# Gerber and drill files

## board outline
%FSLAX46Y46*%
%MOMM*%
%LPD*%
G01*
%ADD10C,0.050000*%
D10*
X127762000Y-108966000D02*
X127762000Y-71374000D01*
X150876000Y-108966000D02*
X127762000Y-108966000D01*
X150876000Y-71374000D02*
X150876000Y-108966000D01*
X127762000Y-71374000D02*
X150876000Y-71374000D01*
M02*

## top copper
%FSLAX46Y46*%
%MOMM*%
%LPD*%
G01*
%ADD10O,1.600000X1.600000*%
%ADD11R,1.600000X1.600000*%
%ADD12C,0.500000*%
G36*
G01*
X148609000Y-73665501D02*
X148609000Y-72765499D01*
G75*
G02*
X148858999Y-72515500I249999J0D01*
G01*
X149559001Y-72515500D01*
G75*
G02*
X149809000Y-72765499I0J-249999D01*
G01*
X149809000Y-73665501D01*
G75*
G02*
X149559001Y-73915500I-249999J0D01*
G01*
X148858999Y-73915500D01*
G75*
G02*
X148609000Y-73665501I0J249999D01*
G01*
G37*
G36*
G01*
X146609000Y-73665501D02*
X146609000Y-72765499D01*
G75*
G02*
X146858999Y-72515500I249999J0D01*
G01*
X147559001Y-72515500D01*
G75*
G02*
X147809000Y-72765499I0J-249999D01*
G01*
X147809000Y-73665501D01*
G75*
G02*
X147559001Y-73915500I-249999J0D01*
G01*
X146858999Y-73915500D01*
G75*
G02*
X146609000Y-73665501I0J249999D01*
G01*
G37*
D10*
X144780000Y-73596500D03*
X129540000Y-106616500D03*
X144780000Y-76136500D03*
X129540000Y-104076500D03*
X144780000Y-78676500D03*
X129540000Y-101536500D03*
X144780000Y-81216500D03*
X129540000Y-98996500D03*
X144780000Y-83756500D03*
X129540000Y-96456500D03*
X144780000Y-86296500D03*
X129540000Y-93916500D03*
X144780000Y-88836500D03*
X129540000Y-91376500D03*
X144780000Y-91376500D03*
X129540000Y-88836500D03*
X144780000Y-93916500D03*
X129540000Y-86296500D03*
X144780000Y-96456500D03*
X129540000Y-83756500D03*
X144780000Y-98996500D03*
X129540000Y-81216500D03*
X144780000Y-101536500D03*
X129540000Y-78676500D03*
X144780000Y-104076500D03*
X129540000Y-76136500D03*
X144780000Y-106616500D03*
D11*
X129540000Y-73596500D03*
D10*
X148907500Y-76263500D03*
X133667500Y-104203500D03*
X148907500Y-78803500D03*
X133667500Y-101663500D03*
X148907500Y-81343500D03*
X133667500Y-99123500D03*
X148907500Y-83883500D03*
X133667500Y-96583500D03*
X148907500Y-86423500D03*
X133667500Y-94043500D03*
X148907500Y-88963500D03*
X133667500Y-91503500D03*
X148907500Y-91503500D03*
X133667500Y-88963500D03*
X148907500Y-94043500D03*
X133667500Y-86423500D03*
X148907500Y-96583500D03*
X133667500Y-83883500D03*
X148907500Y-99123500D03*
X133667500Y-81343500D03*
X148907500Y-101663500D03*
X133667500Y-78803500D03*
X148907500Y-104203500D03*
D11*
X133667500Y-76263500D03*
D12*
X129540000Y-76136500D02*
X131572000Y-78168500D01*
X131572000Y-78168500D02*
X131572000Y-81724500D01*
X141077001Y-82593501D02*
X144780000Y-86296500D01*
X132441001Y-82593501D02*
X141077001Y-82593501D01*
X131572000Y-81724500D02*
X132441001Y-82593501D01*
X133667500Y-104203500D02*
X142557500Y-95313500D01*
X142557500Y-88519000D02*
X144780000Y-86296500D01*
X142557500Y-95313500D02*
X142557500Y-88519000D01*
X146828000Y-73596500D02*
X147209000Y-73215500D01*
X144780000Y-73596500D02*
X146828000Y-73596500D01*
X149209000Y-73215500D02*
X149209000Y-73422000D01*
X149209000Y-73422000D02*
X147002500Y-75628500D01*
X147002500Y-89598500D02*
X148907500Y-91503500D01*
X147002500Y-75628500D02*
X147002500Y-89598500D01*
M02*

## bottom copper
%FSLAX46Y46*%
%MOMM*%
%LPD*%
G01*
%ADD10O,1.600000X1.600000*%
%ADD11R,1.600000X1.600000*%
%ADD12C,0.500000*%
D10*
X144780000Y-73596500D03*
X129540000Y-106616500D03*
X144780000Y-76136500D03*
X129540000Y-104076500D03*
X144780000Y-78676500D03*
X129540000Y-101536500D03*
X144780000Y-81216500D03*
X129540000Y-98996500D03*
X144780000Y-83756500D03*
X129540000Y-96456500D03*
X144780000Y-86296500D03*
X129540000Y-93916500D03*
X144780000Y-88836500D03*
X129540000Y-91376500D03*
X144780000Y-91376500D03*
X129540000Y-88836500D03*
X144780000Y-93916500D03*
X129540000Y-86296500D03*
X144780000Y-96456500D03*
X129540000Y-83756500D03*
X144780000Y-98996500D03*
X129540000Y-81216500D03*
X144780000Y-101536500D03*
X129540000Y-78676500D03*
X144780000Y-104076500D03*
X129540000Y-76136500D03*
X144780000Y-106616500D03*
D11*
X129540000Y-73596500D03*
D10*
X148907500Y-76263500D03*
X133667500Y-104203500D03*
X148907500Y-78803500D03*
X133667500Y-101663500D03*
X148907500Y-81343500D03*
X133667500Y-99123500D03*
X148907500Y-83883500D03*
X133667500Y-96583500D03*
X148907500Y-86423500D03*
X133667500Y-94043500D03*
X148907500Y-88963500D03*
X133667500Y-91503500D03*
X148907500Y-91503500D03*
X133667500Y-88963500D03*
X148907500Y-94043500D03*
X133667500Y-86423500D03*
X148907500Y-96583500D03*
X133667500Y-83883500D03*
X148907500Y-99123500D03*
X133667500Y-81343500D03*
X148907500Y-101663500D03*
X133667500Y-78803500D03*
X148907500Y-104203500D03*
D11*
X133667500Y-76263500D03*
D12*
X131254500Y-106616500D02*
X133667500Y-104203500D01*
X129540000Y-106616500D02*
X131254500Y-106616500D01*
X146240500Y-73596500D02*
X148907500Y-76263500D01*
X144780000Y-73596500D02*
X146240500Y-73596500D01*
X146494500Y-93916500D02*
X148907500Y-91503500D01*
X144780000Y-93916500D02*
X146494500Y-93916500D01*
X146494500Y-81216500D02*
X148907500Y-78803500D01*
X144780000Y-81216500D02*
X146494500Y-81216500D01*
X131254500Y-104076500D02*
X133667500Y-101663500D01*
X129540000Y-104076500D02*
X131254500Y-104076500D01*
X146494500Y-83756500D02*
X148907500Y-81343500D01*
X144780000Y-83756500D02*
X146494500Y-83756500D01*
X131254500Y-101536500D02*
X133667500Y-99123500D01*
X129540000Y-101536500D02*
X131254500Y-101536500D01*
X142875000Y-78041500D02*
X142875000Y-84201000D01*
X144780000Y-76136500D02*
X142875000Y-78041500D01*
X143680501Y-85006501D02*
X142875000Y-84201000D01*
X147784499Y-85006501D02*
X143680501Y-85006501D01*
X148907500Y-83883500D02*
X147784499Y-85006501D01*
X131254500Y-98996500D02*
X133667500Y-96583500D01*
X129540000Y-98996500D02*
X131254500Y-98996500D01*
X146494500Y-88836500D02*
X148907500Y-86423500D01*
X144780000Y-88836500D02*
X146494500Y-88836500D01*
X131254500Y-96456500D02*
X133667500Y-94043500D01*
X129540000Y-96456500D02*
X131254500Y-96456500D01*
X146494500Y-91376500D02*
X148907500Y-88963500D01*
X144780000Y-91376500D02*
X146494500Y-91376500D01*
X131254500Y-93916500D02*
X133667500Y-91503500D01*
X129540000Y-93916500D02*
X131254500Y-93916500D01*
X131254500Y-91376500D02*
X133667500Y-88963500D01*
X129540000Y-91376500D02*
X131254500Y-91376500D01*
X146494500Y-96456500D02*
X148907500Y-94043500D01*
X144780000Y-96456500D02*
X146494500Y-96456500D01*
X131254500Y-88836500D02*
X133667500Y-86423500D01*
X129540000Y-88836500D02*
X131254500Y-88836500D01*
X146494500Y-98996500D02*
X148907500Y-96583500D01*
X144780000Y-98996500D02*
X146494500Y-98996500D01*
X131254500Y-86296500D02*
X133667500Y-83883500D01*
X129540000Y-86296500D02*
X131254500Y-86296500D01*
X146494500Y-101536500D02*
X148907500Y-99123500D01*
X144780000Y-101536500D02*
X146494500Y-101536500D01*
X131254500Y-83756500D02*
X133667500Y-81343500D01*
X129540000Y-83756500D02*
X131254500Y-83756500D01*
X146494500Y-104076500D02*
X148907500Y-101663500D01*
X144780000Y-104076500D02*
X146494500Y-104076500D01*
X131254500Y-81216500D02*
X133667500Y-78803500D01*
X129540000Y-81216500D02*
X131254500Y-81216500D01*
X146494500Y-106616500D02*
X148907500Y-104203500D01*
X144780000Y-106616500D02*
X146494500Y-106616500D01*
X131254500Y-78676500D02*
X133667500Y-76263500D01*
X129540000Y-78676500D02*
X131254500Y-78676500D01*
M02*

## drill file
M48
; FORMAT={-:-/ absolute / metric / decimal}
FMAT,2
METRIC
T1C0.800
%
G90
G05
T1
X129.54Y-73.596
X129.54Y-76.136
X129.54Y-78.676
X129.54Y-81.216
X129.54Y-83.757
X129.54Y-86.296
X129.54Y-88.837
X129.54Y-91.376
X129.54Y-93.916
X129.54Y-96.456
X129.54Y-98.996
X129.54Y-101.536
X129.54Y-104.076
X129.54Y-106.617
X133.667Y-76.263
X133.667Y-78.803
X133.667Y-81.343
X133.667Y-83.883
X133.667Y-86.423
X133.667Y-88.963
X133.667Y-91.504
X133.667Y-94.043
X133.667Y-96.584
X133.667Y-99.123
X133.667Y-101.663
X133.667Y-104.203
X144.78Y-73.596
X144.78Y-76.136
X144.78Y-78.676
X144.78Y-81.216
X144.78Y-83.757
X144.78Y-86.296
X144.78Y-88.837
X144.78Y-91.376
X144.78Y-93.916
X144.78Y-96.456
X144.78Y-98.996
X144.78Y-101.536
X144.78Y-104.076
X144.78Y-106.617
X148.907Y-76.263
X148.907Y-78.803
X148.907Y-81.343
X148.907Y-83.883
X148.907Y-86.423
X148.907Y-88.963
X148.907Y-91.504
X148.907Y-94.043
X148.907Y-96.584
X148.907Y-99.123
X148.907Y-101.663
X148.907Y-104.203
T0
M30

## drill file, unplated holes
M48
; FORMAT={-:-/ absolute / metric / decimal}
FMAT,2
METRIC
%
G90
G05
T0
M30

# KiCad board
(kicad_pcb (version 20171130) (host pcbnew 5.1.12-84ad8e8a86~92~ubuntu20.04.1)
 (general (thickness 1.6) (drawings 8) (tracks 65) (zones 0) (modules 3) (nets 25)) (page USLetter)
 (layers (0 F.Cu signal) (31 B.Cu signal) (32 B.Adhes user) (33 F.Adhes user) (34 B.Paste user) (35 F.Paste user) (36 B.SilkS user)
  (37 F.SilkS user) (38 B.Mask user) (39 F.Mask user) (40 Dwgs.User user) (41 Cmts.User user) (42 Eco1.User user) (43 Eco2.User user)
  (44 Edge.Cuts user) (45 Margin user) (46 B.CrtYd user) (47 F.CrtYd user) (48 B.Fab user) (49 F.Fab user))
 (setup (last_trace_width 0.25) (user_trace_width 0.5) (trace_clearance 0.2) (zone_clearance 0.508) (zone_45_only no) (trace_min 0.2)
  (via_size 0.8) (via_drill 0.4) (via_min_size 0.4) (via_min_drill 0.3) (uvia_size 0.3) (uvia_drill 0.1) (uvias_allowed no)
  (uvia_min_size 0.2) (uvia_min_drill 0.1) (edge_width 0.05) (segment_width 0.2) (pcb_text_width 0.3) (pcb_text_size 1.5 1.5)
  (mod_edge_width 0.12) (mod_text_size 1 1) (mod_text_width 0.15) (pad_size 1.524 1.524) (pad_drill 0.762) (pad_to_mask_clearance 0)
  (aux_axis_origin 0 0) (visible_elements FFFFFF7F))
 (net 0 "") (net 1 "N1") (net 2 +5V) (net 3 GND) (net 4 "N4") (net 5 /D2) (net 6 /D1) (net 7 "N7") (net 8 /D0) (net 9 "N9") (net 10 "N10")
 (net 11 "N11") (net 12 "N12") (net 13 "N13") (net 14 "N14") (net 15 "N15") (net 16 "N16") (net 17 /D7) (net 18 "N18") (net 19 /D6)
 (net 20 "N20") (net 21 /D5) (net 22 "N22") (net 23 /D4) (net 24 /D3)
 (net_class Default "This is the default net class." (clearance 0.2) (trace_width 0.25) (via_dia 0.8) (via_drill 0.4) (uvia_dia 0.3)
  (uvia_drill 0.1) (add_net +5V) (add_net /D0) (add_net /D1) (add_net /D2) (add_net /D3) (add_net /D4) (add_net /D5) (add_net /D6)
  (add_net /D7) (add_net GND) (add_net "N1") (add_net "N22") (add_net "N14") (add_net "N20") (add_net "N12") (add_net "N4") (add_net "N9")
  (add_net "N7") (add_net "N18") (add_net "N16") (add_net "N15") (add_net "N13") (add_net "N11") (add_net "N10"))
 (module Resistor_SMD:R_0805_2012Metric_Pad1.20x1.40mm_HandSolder (layer F.Cu) (at 148.209 73.2155)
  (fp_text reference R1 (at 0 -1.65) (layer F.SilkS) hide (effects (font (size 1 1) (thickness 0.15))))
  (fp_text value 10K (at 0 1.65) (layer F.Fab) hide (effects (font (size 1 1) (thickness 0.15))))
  (pad 2 smd roundrect (at 1 0) (size 1.2 1.4) (layers F.Cu F.Paste F.Mask) (roundrect_rratio 0.2083325) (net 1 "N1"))
  (pad 1 smd roundrect (at -1 0) (size 1.2 1.4) (layers F.Cu F.Paste F.Mask) (roundrect_rratio 0.2083325) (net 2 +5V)))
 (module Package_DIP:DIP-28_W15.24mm (layer F.Cu) (at 129.54 73.5965)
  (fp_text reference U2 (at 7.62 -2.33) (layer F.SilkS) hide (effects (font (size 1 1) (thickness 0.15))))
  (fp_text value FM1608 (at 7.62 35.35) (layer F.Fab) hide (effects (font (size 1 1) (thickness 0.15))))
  (pad 28 thru_hole oval (at 15.24 0) (size 1.6 1.6) (drill 0.8) (layers *.Cu *.Mask) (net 2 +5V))
  (pad 14 thru_hole oval (at 0 33.02) (size 1.6 1.6) (drill 0.8) (layers *.Cu *.Mask) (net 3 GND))
  (pad 27 thru_hole oval (at 15.24 2.54) (size 1.6 1.6) (drill 0.8) (layers *.Cu *.Mask) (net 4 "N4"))
  (pad 13 thru_hole oval (at 0 30.48) (size 1.6 1.6) (drill 0.8) (layers *.Cu *.Mask) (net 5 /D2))
  (pad 26 thru_hole oval (at 15.24 5.08) (size 1.6 1.6) (drill 0.8) (layers *.Cu *.Mask))
  (pad 12 thru_hole oval (at 0 27.94) (size 1.6 1.6) (drill 0.8) (layers *.Cu *.Mask) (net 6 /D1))
  (pad 25 thru_hole oval (at 15.24 7.62) (size 1.6 1.6) (drill 0.8) (layers *.Cu *.Mask) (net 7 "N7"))
  (pad 11 thru_hole oval (at 0 25.4) (size 1.6 1.6) (drill 0.8) (layers *.Cu *.Mask) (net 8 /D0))
  (pad 24 thru_hole oval (at 15.24 10.16) (size 1.6 1.6) (drill 0.8) (layers *.Cu *.Mask) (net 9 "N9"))
  (pad 10 thru_hole oval (at 0 22.86) (size 1.6 1.6) (drill 0.8) (layers *.Cu *.Mask) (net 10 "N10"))
  (pad 23 thru_hole oval (at 15.24 12.7) (size 1.6 1.6) (drill 0.8) (layers *.Cu *.Mask) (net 3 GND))
  (pad 9 thru_hole oval (at 0 20.32) (size 1.6 1.6) (drill 0.8) (layers *.Cu *.Mask) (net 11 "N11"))
  (pad 22 thru_hole oval (at 15.24 15.24) (size 1.6 1.6) (drill 0.8) (layers *.Cu *.Mask) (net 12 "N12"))
  (pad 8 thru_hole oval (at 0 17.78) (size 1.6 1.6) (drill 0.8) (layers *.Cu *.Mask) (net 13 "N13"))
  (pad 21 thru_hole oval (at 15.24 17.78) (size 1.6 1.6) (drill 0.8) (layers *.Cu *.Mask) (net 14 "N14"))
  (pad 7 thru_hole oval (at 0 15.24) (size 1.6 1.6) (drill 0.8) (layers *.Cu *.Mask) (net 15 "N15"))
  (pad 20 thru_hole oval (at 15.24 20.32) (size 1.6 1.6) (drill 0.8) (layers *.Cu *.Mask) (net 1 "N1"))
  (pad 6 thru_hole oval (at 0 12.7) (size 1.6 1.6) (drill 0.8) (layers *.Cu *.Mask) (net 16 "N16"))
  (pad 19 thru_hole oval (at 15.24 22.86) (size 1.6 1.6) (drill 0.8) (layers *.Cu *.Mask) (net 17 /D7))
  (pad 5 thru_hole oval (at 0 10.16) (size 1.6 1.6) (drill 0.8) (layers *.Cu *.Mask) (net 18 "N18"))
  (pad 18 thru_hole oval (at 15.24 25.4) (size 1.6 1.6) (drill 0.8) (layers *.Cu *.Mask) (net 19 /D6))
  (pad 4 thru_hole oval (at 0 7.62) (size 1.6 1.6) (drill 0.8) (layers *.Cu *.Mask) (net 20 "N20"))
  (pad 17 thru_hole oval (at 15.24 27.94) (size 1.6 1.6) (drill 0.8) (layers *.Cu *.Mask) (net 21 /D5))
  (pad 3 thru_hole oval (at 0 5.08) (size 1.6 1.6) (drill 0.8) (layers *.Cu *.Mask) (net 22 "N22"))
  (pad 16 thru_hole oval (at 15.24 30.48) (size 1.6 1.6) (drill 0.8) (layers *.Cu *.Mask) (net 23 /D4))
  (pad 2 thru_hole oval (at 0 2.54) (size 1.6 1.6) (drill 0.8) (layers *.Cu *.Mask) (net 3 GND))
  (pad 15 thru_hole oval (at 15.24 33.02) (size 1.6 1.6) (drill 0.8) (layers *.Cu *.Mask) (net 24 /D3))
  (pad 1 thru_hole rect (at 0 0) (size 1.6 1.6) (drill 0.8) (layers *.Cu *.Mask)))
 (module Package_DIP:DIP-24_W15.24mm (layer F.Cu) (at 133.6675 76.2635)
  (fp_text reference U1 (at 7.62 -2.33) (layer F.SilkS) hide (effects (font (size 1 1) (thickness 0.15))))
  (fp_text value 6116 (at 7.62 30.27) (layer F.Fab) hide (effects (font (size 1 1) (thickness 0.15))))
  (pad 24 thru_hole oval (at 15.24 0) (size 1.6 1.6) (drill 0.8) (layers *.Cu *.Mask) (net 2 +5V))
  (pad 12 thru_hole oval (at 0 27.94) (size 1.6 1.6) (drill 0.8) (layers *.Cu *.Mask) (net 3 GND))
  (pad 23 thru_hole oval (at 15.24 2.54) (size 1.6 1.6) (drill 0.8) (layers *.Cu *.Mask) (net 7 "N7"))
  (pad 11 thru_hole oval (at 0 25.4) (size 1.6 1.6) (drill 0.8) (layers *.Cu *.Mask) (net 5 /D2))
  (pad 22 thru_hole oval (at 15.24 5.08) (size 1.6 1.6) (drill 0.8) (layers *.Cu *.Mask) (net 9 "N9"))
  (pad 10 thru_hole oval (at 0 22.86) (size 1.6 1.6) (drill 0.8) (layers *.Cu *.Mask) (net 6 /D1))
  (pad 21 thru_hole oval (at 15.24 7.62) (size 1.6 1.6) (drill 0.8) (layers *.Cu *.Mask) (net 4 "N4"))
  (pad 9 thru_hole oval (at 0 20.32) (size 1.6 1.6) (drill 0.8) (layers *.Cu *.Mask) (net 8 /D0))
  (pad 20 thru_hole oval (at 15.24 10.16) (size 1.6 1.6) (drill 0.8) (layers *.Cu *.Mask) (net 12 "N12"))
  (pad 8 thru_hole oval (at 0 17.78) (size 1.6 1.6) (drill 0.8) (layers *.Cu *.Mask) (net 10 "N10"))
  (pad 19 thru_hole oval (at 15.24 12.7) (size 1.6 1.6) (drill 0.8) (layers *.Cu *.Mask) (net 14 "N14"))
  (pad 7 thru_hole oval (at 0 15.24) (size 1.6 1.6) (drill 0.8) (layers *.Cu *.Mask) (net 11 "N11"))
  (pad 18 thru_hole oval (at 15.24 15.24) (size 1.6 1.6) (drill 0.8) (layers *.Cu *.Mask) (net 1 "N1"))
  (pad 6 thru_hole oval (at 0 12.7) (size 1.6 1.6) (drill 0.8) (layers *.Cu *.Mask) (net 13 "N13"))
  (pad 17 thru_hole oval (at 15.24 17.78) (size 1.6 1.6) (drill 0.8) (layers *.Cu *.Mask) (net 17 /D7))
  (pad 5 thru_hole oval (at 0 10.16) (size 1.6 1.6) (drill 0.8) (layers *.Cu *.Mask) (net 15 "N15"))
  (pad 16 thru_hole oval (at 15.24 20.32) (size 1.6 1.6) (drill 0.8) (layers *.Cu *.Mask) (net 19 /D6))
  (pad 4 thru_hole oval (at 0 7.62) (size 1.6 1.6) (drill 0.8) (layers *.Cu *.Mask) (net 16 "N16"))
  (pad 15 thru_hole oval (at 15.24 22.86) (size 1.6 1.6) (drill 0.8) (layers *.Cu *.Mask) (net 21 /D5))
  (pad 3 thru_hole oval (at 0 5.08) (size 1.6 1.6) (drill 0.8) (layers *.Cu *.Mask) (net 18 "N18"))
  (pad 14 thru_hole oval (at 15.24 25.4) (size 1.6 1.6) (drill 0.8) (layers *.Cu *.Mask) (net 23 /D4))
  (pad 2 thru_hole oval (at 0 2.54) (size 1.6 1.6) (drill 0.8) (layers *.Cu *.Mask) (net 20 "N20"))
  (pad 13 thru_hole oval (at 15.24 27.94) (size 1.6 1.6) (drill 0.8) (layers *.Cu *.Mask) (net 24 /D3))
  (pad 1 thru_hole rect (at 0 0) (size 1.6 1.6) (drill 0.8) (layers *.Cu *.Mask) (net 22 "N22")))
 (gr_line (start 127.762 108.966) (end 127.762 71.374) (layer Edge.Cuts) (width 0.05))
 (gr_line (start 150.876 108.966) (end 127.762 108.966) (layer Edge.Cuts) (width 0.05))
 (gr_line (start 150.876 71.374) (end 150.876 108.966) (layer Edge.Cuts) (width 0.05))
 (gr_line (start 127.762 71.374) (end 150.876 71.374) (layer Edge.Cuts) (width 0.05))
 (segment (start 131.2545 106.6165) (end 133.6675 104.2035) (width 0.5) (layer B.Cu) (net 3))
 (segment (start 129.54 106.6165) (end 131.2545 106.6165) (width 0.5) (layer B.Cu) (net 3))
 (segment (start 129.54 76.1365) (end 131.572 78.1685) (width 0.5) (layer F.Cu) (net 3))
 (segment (start 131.572 78.1685) (end 131.572 81.7245) (width 0.5) (layer F.Cu) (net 3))
 (segment (start 141.077001 82.593501) (end 144.78 86.2965) (width 0.5) (layer F.Cu) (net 3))
 (segment (start 132.441001 82.593501) (end 141.077001 82.593501) (width 0.5) (layer F.Cu) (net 3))
 (segment (start 131.572 81.7245) (end 132.441001 82.593501) (width 0.5) (layer F.Cu) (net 3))
 (segment (start 133.6675 104.2035) (end 142.5575 95.3135) (width 0.5) (layer F.Cu) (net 3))
 (segment (start 142.5575 88.519) (end 144.78 86.2965) (width 0.5) (layer F.Cu) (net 3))
 (segment (start 142.5575 95.3135) (end 142.5575 88.519) (width 0.5) (layer F.Cu) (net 3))
 (segment (start 146.828 73.5965) (end 147.209 73.2155) (width 0.5) (layer F.Cu) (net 2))
 (segment (start 144.78 73.5965) (end 146.828 73.5965) (width 0.5) (layer F.Cu) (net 2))
 (segment (start 146.2405 73.5965) (end 148.9075 76.2635) (width 0.5) (layer B.Cu) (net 2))
 (segment (start 144.78 73.5965) (end 146.2405 73.5965) (width 0.5) (layer B.Cu) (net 2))
 (segment (start 146.4945 93.9165) (end 148.9075 91.5035) (width 0.5) (layer B.Cu) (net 1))
 (segment (start 144.78 93.9165) (end 146.4945 93.9165) (width 0.5) (layer B.Cu) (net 1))
 (segment (start 149.209 73.2155) (end 149.209 73.422) (width 0.5) (layer F.Cu) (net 1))
 (segment (start 149.209 73.422) (end 147.0025 75.6285) (width 0.5) (layer F.Cu) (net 1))
 (segment (start 147.0025 89.5985) (end 148.9075 91.5035) (width 0.5) (layer F.Cu) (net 1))
 (segment (start 147.0025 75.6285) (end 147.0025 89.5985) (width 0.5) (layer F.Cu) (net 1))
 (segment (start 146.4945 81.2165) (end 148.9075 78.8035) (width 0.5) (layer B.Cu) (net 7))
 (segment (start 144.78 81.2165) (end 146.4945 81.2165) (width 0.5) (layer B.Cu) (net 7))
 (segment (start 131.2545 104.0765) (end 133.6675 101.6635) (width 0.5) (layer B.Cu) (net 5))
 (segment (start 129.54 104.0765) (end 131.2545 104.0765) (width 0.5) (layer B.Cu) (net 5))
 (segment (start 146.4945 83.7565) (end 148.9075 81.3435) (width 0.5) (layer B.Cu) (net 9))
 (segment (start 144.78 83.7565) (end 146.4945 83.7565) (width 0.5) (layer B.Cu) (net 9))
 (segment (start 131.2545 101.5365) (end 133.6675 99.1235) (width 0.5) (layer B.Cu) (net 6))
 (segment (start 129.54 101.5365) (end 131.2545 101.5365) (width 0.5) (layer B.Cu) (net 6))
 (segment (start 142.875 78.0415) (end 142.875 84.201) (width 0.5) (layer B.Cu) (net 4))
 (segment (start 144.78 76.1365) (end 142.875 78.0415) (width 0.5) (layer B.Cu) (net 4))
 (segment (start 143.680501 85.006501) (end 142.875 84.201) (width 0.5) (layer B.Cu) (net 4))
 (segment (start 147.784499 85.006501) (end 143.680501 85.006501) (width 0.5) (layer B.Cu) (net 4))
 (segment (start 148.9075 83.8835) (end 147.784499 85.006501) (width 0.5) (layer B.Cu) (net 4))
 (segment (start 131.2545 98.9965) (end 133.6675 96.5835) (width 0.5) (layer B.Cu) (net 8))
 (segment (start 129.54 98.9965) (end 131.2545 98.9965) (width 0.5) (layer B.Cu) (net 8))
 (segment (start 146.4945 88.8365) (end 148.9075 86.4235) (width 0.5) (layer B.Cu) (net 12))
 (segment (start 144.78 88.8365) (end 146.4945 88.8365) (width 0.5) (layer B.Cu) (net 12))
 (segment (start 131.2545 96.4565) (end 133.6675 94.0435) (width 0.5) (layer B.Cu) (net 10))
 (segment (start 129.54 96.4565) (end 131.2545 96.4565) (width 0.5) (layer B.Cu) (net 10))
 (segment (start 146.4945 91.3765) (end 148.9075 88.9635) (width 0.5) (layer B.Cu) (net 14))
 (segment (start 144.78 91.3765) (end 146.4945 91.3765) (width 0.5) (layer B.Cu) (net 14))
 (segment (start 131.2545 93.9165) (end 133.6675 91.5035) (width 0.5) (layer B.Cu) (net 11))
 (segment (start 129.54 93.9165) (end 131.2545 93.9165) (width 0.5) (layer B.Cu) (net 11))
 (segment (start 131.2545 91.3765) (end 133.6675 88.9635) (width 0.5) (layer B.Cu) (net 13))
 (segment (start 129.54 91.3765) (end 131.2545 91.3765) (width 0.5) (layer B.Cu) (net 13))
 (segment (start 146.4945 96.4565) (end 148.9075 94.0435) (width 0.5) (layer B.Cu) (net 17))
 (segment (start 144.78 96.4565) (end 146.4945 96.4565) (width 0.5) (layer B.Cu) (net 17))
 (segment (start 131.2545 88.8365) (end 133.6675 86.4235) (width 0.5) (layer B.Cu) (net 15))
 (segment (start 129.54 88.8365) (end 131.2545 88.8365) (width 0.5) (layer B.Cu) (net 15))
 (segment (start 146.4945 98.9965) (end 148.9075 96.5835) (width 0.5) (layer B.Cu) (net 19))
 (segment (start 144.78 98.9965) (end 146.4945 98.9965) (width 0.5) (layer B.Cu) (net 19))
 (segment (start 131.2545 86.2965) (end 133.6675 83.8835) (width 0.5) (layer B.Cu) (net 16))
 (segment (start 129.54 86.2965) (end 131.2545 86.2965) (width 0.5) (layer B.Cu) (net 16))
 (segment (start 146.4945 101.5365) (end 148.9075 99.1235) (width 0.5) (layer B.Cu) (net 21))
 (segment (start 144.78 101.5365) (end 146.4945 101.5365) (width 0.5) (layer B.Cu) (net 21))
 (segment (start 131.2545 83.7565) (end 133.6675 81.3435) (width 0.5) (layer B.Cu) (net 18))
 (segment (start 129.54 83.7565) (end 131.2545 83.7565) (width 0.5) (layer B.Cu) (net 18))
 (segment (start 146.4945 104.0765) (end 148.9075 101.6635) (width 0.5) (layer B.Cu) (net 23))
 (segment (start 144.78 104.0765) (end 146.4945 104.0765) (width 0.5) (layer B.Cu) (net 23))
 (segment (start 131.2545 81.2165) (end 133.6675 78.8035) (width 0.5) (layer B.Cu) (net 20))
 (segment (start 129.54 81.2165) (end 131.2545 81.2165) (width 0.5) (layer B.Cu) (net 20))
 (segment (start 146.4945 106.6165) (end 148.9075 104.2035) (width 0.5) (layer B.Cu) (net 24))
 (segment (start 144.78 106.6165) (end 146.4945 106.6165) (width 0.5) (layer B.Cu) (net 24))
 (segment (start 131.2545 78.6765) (end 133.6675 76.2635) (width 0.5) (layer B.Cu) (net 22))
 (segment (start 129.54 78.6765) (end 131.2545 78.6765) (width 0.5) (layer B.Cu) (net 22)))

